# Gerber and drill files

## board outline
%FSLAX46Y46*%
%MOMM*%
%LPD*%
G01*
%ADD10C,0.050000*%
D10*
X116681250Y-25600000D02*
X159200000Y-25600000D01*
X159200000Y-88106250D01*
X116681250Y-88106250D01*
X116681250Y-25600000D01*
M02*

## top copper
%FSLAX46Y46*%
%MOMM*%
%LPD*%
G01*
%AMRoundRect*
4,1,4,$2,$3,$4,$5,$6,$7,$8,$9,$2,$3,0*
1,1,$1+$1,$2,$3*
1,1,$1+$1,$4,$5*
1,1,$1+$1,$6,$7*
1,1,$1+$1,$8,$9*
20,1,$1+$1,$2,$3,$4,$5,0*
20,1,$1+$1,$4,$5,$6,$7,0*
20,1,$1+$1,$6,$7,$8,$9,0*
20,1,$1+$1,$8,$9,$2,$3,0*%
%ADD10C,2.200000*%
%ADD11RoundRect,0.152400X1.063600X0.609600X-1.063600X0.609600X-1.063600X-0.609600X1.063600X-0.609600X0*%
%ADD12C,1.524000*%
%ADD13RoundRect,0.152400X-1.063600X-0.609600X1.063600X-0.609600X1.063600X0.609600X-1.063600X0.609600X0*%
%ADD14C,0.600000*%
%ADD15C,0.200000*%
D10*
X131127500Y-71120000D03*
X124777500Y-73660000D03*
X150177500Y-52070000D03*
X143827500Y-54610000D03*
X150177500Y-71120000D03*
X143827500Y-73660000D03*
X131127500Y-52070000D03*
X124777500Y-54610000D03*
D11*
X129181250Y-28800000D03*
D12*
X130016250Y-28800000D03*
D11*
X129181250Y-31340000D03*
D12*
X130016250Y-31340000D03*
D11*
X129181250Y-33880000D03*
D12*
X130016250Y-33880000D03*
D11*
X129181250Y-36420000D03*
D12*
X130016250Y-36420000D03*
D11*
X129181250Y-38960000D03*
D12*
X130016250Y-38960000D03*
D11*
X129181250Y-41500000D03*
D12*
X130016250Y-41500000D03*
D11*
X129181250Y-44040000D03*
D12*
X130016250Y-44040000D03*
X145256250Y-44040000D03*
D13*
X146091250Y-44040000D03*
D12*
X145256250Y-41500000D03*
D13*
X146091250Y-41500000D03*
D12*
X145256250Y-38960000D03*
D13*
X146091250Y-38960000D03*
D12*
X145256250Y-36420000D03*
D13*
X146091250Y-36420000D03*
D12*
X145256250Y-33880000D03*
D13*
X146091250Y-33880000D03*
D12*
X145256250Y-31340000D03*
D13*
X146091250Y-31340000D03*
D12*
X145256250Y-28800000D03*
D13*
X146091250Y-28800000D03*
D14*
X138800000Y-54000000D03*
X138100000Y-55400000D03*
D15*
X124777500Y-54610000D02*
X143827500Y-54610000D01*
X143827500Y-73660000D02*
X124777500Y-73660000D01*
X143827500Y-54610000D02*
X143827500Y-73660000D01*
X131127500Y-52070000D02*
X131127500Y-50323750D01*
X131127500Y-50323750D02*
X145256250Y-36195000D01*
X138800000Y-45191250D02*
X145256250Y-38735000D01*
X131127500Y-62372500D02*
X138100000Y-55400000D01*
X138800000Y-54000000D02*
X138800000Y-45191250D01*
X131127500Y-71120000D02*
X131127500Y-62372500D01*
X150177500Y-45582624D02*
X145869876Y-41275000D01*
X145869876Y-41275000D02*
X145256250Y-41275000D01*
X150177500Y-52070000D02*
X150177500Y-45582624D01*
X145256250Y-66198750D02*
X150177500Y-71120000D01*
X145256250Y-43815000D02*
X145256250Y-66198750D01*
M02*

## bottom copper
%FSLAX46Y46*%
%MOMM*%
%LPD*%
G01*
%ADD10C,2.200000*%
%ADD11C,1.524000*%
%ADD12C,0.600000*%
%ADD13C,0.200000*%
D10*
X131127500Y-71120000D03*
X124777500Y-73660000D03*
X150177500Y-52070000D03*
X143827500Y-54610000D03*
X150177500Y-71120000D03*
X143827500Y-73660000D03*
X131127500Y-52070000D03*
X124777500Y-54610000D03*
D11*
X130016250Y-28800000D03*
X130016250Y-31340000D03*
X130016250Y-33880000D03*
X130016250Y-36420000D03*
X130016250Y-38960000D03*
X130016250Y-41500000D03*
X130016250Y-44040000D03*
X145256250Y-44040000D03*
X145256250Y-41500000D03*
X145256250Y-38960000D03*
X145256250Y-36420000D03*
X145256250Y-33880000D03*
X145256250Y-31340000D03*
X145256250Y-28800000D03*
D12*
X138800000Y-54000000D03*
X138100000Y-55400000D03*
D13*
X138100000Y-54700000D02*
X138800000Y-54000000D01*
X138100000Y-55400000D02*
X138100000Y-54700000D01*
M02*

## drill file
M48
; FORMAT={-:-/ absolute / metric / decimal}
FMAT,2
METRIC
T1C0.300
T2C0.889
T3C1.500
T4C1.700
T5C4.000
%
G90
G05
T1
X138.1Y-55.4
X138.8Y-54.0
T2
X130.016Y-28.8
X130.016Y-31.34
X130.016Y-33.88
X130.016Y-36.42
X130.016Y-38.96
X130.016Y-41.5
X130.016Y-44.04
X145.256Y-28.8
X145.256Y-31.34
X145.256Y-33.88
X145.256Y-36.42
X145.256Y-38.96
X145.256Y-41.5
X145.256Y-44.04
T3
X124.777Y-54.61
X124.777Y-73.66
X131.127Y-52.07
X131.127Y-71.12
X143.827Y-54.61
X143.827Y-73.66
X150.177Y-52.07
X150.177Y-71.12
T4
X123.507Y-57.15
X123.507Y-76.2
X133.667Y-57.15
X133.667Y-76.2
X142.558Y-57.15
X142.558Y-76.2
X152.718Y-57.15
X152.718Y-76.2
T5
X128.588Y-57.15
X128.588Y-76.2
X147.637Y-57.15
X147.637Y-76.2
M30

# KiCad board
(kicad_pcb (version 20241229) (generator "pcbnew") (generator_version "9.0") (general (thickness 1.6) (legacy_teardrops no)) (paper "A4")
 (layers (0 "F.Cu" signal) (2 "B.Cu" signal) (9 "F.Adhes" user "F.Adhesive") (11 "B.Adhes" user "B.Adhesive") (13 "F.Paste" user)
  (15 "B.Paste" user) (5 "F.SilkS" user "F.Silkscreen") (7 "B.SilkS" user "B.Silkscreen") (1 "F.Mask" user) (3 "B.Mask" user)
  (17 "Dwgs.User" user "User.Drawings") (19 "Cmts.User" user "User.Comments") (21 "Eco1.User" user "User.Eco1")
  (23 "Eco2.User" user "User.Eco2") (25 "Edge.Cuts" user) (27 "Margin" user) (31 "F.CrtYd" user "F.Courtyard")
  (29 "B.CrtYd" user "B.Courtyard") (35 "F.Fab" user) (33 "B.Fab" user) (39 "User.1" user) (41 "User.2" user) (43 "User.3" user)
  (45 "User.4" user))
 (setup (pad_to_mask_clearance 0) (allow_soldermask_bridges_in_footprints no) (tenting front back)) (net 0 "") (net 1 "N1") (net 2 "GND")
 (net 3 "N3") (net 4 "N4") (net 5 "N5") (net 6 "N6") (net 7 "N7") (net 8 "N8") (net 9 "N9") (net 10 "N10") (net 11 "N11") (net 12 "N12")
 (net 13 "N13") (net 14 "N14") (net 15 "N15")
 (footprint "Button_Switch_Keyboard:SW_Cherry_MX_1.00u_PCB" (layer "F.Cu") (at 131.1275 71.12)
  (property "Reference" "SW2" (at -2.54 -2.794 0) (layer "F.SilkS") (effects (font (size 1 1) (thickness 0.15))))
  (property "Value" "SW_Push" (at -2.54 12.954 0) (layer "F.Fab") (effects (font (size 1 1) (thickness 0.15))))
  (pad "" np_thru_hole circle (at -7.62 5.08) (size 1.7 1.7) (drill 1.7) (layers "*.Cu" "*.Mask"))
  (pad "" np_thru_hole circle (at -2.54 5.08) (size 4 4) (drill 4) (layers "*.Cu" "*.Mask"))
  (pad "" np_thru_hole circle (at 2.54 5.08) (size 1.7 1.7) (drill 1.7) (layers "*.Cu" "*.Mask"))
  (pad "1" thru_hole circle (at 0 0) (size 2.2 2.2) (drill 1.5) (layers "*.Cu" "*.Mask") (remove_unused_layers no) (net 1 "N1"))
  (pad "2" thru_hole circle (at -6.35 2.54) (size 2.2 2.2) (drill 1.5) (layers "*.Cu" "*.Mask") (remove_unused_layers no) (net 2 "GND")))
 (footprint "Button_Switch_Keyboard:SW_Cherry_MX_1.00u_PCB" (layer "F.Cu") (at 150.1775 52.07)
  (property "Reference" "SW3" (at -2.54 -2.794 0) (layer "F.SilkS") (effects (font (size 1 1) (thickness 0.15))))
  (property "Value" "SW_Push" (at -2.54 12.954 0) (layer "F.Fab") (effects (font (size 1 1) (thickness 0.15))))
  (pad "" np_thru_hole circle (at -7.62 5.08) (size 1.7 1.7) (drill 1.7) (layers "*.Cu" "*.Mask"))
  (pad "" np_thru_hole circle (at -2.54 5.08) (size 4 4) (drill 4) (layers "*.Cu" "*.Mask"))
  (pad "" np_thru_hole circle (at 2.54 5.08) (size 1.7 1.7) (drill 1.7) (layers "*.Cu" "*.Mask"))
  (pad "1" thru_hole circle (at 0 0) (size 2.2 2.2) (drill 1.5) (layers "*.Cu" "*.Mask") (remove_unused_layers no) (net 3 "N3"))
  (pad "2" thru_hole circle (at -6.35 2.54) (size 2.2 2.2) (drill 1.5) (layers "*.Cu" "*.Mask") (remove_unused_layers no) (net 2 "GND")))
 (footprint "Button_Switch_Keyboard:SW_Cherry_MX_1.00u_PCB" (layer "F.Cu") (at 150.1775 71.12)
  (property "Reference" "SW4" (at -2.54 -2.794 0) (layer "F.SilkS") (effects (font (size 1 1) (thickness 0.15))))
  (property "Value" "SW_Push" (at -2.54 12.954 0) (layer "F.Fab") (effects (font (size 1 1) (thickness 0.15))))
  (pad "" np_thru_hole circle (at -7.62 5.08) (size 1.7 1.7) (drill 1.7) (layers "*.Cu" "*.Mask"))
  (pad "" np_thru_hole circle (at -2.54 5.08) (size 4 4) (drill 4) (layers "*.Cu" "*.Mask"))
  (pad "" np_thru_hole circle (at 2.54 5.08) (size 1.7 1.7) (drill 1.7) (layers "*.Cu" "*.Mask"))
  (pad "1" thru_hole circle (at 0 0) (size 2.2 2.2) (drill 1.5) (layers "*.Cu" "*.Mask") (remove_unused_layers no) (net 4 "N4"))
  (pad "2" thru_hole circle (at -6.35 2.54) (size 2.2 2.2) (drill 1.5) (layers "*.Cu" "*.Mask") (remove_unused_layers no) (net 2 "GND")))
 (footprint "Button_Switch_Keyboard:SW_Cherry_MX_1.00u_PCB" (layer "F.Cu") (at 131.1275 52.07)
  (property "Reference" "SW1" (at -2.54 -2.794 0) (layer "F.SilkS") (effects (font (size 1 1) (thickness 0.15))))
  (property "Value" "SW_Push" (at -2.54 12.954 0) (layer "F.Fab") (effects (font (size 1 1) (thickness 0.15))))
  (pad "" np_thru_hole circle (at -7.62 5.08) (size 1.7 1.7) (drill 1.7) (layers "*.Cu" "*.Mask"))
  (pad "" np_thru_hole circle (at -2.54 5.08) (size 4 4) (drill 4) (layers "*.Cu" "*.Mask"))
  (pad "" np_thru_hole circle (at 2.54 5.08) (size 1.7 1.7) (drill 1.7) (layers "*.Cu" "*.Mask"))
  (pad "1" thru_hole circle (at 0 0) (size 2.2 2.2) (drill 1.5) (layers "*.Cu" "*.Mask") (remove_unused_layers no) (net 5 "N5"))
  (pad "2" thru_hole circle (at -6.35 2.54) (size 2.2 2.2) (drill 1.5) (layers "*.Cu" "*.Mask") (remove_unused_layers no) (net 2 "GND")))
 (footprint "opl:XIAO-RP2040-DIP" (layer "F.Cu") (at 137.63625 36.42)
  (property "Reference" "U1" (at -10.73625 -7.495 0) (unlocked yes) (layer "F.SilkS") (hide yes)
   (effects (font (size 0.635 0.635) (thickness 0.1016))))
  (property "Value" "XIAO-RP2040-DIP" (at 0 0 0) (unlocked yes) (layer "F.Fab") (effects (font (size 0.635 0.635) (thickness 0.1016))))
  (pad "1" smd roundrect (at -8.455 -7.62 180) (size 2.432 1.524) (layers "F.Cu" "F.Mask") (roundrect_rratio 0.1) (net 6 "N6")
   (thermal_bridge_angle 45))
  (pad "1" thru_hole circle (at -7.62 -7.62 180) (size 1.524 1.524) (drill 0.889) (layers "*.Cu" "*.Mask") (remove_unused_layers no)
   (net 6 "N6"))
  (pad "2" smd roundrect (at -8.455 -5.08 180) (size 2.432 1.524) (layers "F.Cu" "F.Mask") (roundrect_rratio 0.1) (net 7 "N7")
   (thermal_bridge_angle 45))
  (pad "2" thru_hole circle (at -7.62 -5.08 180) (size 1.524 1.524) (drill 0.889) (layers "*.Cu" "*.Mask") (remove_unused_layers no)
   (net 7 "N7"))
  (pad "3" smd roundrect (at -8.455 -2.54 180) (size 2.432 1.524) (layers "F.Cu" "F.Mask") (roundrect_rratio 0.1) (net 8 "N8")
   (thermal_bridge_angle 45))
  (pad "3" thru_hole circle (at -7.62 -2.54 180) (size 1.524 1.524) (drill 0.889) (layers "*.Cu" "*.Mask") (remove_unused_layers no)
   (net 8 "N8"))
  (pad "4" smd roundrect (at -8.455 0 180) (size 2.432 1.524) (layers "F.Cu" "F.Mask") (roundrect_rratio 0.1) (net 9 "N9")
   (thermal_bridge_angle 45))
  (pad "4" thru_hole circle (at -7.62 0 180) (size 1.524 1.524) (drill 0.889) (layers "*.Cu" "*.Mask") (remove_unused_layers no)
   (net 9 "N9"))
  (pad "5" smd roundrect (at -8.455 2.54 180) (size 2.432 1.524) (layers "F.Cu" "F.Mask") (roundrect_rratio 0.1) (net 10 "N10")
   (thermal_bridge_angle 45))
  (pad "5" thru_hole circle (at -7.62 2.54 180) (size 1.524 1.524) (drill 0.889) (layers "*.Cu" "*.Mask") (remove_unused_layers no)
   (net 10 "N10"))
  (pad "6" smd roundrect (at -8.455 5.08 180) (size 2.432 1.524) (layers "F.Cu" "F.Mask") (roundrect_rratio 0.1) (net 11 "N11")
   (thermal_bridge_angle 45))
  (pad "6" thru_hole circle (at -7.62 5.08 180) (size 1.524 1.524) (drill 0.889) (layers "*.Cu" "*.Mask") (remove_unused_layers no)
   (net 11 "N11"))
  (pad "7" smd roundrect (at -8.455 7.62 180) (size 2.432 1.524) (layers "F.Cu" "F.Mask") (roundrect_rratio 0.1) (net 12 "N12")
   (thermal_bridge_angle 45))
  (pad "7" thru_hole circle (at -7.62 7.62 180) (size 1.524 1.524) (drill 0.889) (layers "*.Cu" "*.Mask") (remove_unused_layers no)
   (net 12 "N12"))
  (pad "8" thru_hole circle (at 7.62 7.62) (size 1.524 1.524) (drill 0.889) (layers "*.Cu" "*.Mask") (remove_unused_layers no) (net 4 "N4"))
  (pad "8" smd roundrect (at 8.455 7.62) (size 2.432 1.524) (layers "F.Cu" "F.Mask") (roundrect_rratio 0.1) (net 4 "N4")
   (thermal_bridge_angle 45))
  (pad "9" thru_hole circle (at 7.62 5.08) (size 1.524 1.524) (drill 0.889) (layers "*.Cu" "*.Mask") (remove_unused_layers no) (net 3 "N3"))
  (pad "9" smd roundrect (at 8.455 5.08) (size 2.432 1.524) (layers "F.Cu" "F.Mask") (roundrect_rratio 0.1) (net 3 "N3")
   (thermal_bridge_angle 45))
  (pad "10" thru_hole circle (at 7.62 2.54) (size 1.524 1.524) (drill 0.889) (layers "*.Cu" "*.Mask") (remove_unused_layers no) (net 1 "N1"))
  (pad "10" smd roundrect (at 8.455 2.54) (size 2.432 1.524) (layers "F.Cu" "F.Mask") (roundrect_rratio 0.1) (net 1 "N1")
   (thermal_bridge_angle 45))
  (pad "11" thru_hole circle (at 7.62 0) (size 1.524 1.524) (drill 0.889) (layers "*.Cu" "*.Mask") (remove_unused_layers no) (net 5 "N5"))
  (pad "11" smd roundrect (at 8.455 0) (size 2.432 1.524) (layers "F.Cu" "F.Mask") (roundrect_rratio 0.1) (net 5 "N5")
   (thermal_bridge_angle 45))
  (pad "12" thru_hole circle (at 7.62 -2.54) (size 1.524 1.524) (drill 0.889) (layers "*.Cu" "*.Mask") (remove_unused_layers no)
   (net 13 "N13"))
  (pad "12" smd roundrect (at 8.455 -2.54) (size 2.432 1.524) (layers "F.Cu" "F.Mask") (roundrect_rratio 0.1) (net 13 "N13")
   (thermal_bridge_angle 45))
  (pad "13" thru_hole circle (at 7.62 -5.08) (size 1.524 1.524) (drill 0.889) (layers "*.Cu" "*.Mask") (remove_unused_layers no)
   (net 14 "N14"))
  (pad "13" smd roundrect (at 8.455 -5.08) (size 2.432 1.524) (layers "F.Cu" "F.Mask") (roundrect_rratio 0.1) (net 14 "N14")
   (thermal_bridge_angle 45))
  (pad "14" thru_hole circle (at 7.62 -7.62) (size 1.524 1.524) (drill 0.889) (layers "*.Cu" "*.Mask") (remove_unused_layers no)
   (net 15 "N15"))
  (pad "14" smd roundrect (at 8.455 -7.62) (size 2.432 1.524) (layers "F.Cu" "F.Mask") (roundrect_rratio 0.1) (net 15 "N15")
   (thermal_bridge_angle 45)))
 (gr_rect (start 116.68125 25.6) (end 159.2 88.10625) (stroke (width 0.05) (type default)) (fill no) (layer "Edge.Cuts"))
 (segment (start 124.7775 54.61) (end 143.8275 54.61) (width 0.2) (layer "F.Cu") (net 2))
 (segment (start 143.8275 73.66) (end 124.7775 73.66) (width 0.2) (layer "F.Cu") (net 2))
 (segment (start 143.8275 54.61) (end 143.8275 73.66) (width 0.2) (layer "F.Cu") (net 2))
 (segment (start 131.1275 52.07) (end 131.1275 50.32375) (width 0.2) (layer "F.Cu") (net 5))
 (segment (start 131.1275 50.32375) (end 145.25625 36.195) (width 0.2) (layer "F.Cu") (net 5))
 (segment (start 138.8 45.19125) (end 145.25625 38.735) (width 0.2) (layer "F.Cu") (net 1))
 (segment (start 131.1275 62.3725) (end 138.1 55.4) (width 0.2) (layer "F.Cu") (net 1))
 (segment (start 138.8 54) (end 138.8 45.19125) (width 0.2) (layer "F.Cu") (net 1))
 (segment (start 131.1275 71.12) (end 131.1275 62.3725) (width 0.2) (layer "F.Cu") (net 1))
 (via (at 138.8 54) (size 0.6) (drill 0.3) (layers "F.Cu" "B.Cu") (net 1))
 (via (at 138.1 55.4) (size 0.6) (drill 0.3) (layers "F.Cu" "B.Cu") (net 1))
 (segment (start 138.1 54.7) (end 138.8 54) (width 0.2) (layer "B.Cu") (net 1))
 (segment (start 138.1 55.4) (end 138.1 54.7) (width 0.2) (layer "B.Cu") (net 1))
 (segment (start 150.1775 45.582624) (end 145.869876 41.275) (width 0.2) (layer "F.Cu") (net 3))
 (segment (start 145.869876 41.275) (end 145.25625 41.275) (width 0.2) (layer "F.Cu") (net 3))
 (segment (start 150.1775 52.07) (end 150.1775 45.582624) (width 0.2) (layer "F.Cu") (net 3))
 (segment (start 145.25625 66.19875) (end 150.1775 71.12) (width 0.2) (layer "F.Cu") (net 4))
 (segment (start 145.25625 43.815) (end 145.25625 66.19875) (width 0.2) (layer "F.Cu") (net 4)))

